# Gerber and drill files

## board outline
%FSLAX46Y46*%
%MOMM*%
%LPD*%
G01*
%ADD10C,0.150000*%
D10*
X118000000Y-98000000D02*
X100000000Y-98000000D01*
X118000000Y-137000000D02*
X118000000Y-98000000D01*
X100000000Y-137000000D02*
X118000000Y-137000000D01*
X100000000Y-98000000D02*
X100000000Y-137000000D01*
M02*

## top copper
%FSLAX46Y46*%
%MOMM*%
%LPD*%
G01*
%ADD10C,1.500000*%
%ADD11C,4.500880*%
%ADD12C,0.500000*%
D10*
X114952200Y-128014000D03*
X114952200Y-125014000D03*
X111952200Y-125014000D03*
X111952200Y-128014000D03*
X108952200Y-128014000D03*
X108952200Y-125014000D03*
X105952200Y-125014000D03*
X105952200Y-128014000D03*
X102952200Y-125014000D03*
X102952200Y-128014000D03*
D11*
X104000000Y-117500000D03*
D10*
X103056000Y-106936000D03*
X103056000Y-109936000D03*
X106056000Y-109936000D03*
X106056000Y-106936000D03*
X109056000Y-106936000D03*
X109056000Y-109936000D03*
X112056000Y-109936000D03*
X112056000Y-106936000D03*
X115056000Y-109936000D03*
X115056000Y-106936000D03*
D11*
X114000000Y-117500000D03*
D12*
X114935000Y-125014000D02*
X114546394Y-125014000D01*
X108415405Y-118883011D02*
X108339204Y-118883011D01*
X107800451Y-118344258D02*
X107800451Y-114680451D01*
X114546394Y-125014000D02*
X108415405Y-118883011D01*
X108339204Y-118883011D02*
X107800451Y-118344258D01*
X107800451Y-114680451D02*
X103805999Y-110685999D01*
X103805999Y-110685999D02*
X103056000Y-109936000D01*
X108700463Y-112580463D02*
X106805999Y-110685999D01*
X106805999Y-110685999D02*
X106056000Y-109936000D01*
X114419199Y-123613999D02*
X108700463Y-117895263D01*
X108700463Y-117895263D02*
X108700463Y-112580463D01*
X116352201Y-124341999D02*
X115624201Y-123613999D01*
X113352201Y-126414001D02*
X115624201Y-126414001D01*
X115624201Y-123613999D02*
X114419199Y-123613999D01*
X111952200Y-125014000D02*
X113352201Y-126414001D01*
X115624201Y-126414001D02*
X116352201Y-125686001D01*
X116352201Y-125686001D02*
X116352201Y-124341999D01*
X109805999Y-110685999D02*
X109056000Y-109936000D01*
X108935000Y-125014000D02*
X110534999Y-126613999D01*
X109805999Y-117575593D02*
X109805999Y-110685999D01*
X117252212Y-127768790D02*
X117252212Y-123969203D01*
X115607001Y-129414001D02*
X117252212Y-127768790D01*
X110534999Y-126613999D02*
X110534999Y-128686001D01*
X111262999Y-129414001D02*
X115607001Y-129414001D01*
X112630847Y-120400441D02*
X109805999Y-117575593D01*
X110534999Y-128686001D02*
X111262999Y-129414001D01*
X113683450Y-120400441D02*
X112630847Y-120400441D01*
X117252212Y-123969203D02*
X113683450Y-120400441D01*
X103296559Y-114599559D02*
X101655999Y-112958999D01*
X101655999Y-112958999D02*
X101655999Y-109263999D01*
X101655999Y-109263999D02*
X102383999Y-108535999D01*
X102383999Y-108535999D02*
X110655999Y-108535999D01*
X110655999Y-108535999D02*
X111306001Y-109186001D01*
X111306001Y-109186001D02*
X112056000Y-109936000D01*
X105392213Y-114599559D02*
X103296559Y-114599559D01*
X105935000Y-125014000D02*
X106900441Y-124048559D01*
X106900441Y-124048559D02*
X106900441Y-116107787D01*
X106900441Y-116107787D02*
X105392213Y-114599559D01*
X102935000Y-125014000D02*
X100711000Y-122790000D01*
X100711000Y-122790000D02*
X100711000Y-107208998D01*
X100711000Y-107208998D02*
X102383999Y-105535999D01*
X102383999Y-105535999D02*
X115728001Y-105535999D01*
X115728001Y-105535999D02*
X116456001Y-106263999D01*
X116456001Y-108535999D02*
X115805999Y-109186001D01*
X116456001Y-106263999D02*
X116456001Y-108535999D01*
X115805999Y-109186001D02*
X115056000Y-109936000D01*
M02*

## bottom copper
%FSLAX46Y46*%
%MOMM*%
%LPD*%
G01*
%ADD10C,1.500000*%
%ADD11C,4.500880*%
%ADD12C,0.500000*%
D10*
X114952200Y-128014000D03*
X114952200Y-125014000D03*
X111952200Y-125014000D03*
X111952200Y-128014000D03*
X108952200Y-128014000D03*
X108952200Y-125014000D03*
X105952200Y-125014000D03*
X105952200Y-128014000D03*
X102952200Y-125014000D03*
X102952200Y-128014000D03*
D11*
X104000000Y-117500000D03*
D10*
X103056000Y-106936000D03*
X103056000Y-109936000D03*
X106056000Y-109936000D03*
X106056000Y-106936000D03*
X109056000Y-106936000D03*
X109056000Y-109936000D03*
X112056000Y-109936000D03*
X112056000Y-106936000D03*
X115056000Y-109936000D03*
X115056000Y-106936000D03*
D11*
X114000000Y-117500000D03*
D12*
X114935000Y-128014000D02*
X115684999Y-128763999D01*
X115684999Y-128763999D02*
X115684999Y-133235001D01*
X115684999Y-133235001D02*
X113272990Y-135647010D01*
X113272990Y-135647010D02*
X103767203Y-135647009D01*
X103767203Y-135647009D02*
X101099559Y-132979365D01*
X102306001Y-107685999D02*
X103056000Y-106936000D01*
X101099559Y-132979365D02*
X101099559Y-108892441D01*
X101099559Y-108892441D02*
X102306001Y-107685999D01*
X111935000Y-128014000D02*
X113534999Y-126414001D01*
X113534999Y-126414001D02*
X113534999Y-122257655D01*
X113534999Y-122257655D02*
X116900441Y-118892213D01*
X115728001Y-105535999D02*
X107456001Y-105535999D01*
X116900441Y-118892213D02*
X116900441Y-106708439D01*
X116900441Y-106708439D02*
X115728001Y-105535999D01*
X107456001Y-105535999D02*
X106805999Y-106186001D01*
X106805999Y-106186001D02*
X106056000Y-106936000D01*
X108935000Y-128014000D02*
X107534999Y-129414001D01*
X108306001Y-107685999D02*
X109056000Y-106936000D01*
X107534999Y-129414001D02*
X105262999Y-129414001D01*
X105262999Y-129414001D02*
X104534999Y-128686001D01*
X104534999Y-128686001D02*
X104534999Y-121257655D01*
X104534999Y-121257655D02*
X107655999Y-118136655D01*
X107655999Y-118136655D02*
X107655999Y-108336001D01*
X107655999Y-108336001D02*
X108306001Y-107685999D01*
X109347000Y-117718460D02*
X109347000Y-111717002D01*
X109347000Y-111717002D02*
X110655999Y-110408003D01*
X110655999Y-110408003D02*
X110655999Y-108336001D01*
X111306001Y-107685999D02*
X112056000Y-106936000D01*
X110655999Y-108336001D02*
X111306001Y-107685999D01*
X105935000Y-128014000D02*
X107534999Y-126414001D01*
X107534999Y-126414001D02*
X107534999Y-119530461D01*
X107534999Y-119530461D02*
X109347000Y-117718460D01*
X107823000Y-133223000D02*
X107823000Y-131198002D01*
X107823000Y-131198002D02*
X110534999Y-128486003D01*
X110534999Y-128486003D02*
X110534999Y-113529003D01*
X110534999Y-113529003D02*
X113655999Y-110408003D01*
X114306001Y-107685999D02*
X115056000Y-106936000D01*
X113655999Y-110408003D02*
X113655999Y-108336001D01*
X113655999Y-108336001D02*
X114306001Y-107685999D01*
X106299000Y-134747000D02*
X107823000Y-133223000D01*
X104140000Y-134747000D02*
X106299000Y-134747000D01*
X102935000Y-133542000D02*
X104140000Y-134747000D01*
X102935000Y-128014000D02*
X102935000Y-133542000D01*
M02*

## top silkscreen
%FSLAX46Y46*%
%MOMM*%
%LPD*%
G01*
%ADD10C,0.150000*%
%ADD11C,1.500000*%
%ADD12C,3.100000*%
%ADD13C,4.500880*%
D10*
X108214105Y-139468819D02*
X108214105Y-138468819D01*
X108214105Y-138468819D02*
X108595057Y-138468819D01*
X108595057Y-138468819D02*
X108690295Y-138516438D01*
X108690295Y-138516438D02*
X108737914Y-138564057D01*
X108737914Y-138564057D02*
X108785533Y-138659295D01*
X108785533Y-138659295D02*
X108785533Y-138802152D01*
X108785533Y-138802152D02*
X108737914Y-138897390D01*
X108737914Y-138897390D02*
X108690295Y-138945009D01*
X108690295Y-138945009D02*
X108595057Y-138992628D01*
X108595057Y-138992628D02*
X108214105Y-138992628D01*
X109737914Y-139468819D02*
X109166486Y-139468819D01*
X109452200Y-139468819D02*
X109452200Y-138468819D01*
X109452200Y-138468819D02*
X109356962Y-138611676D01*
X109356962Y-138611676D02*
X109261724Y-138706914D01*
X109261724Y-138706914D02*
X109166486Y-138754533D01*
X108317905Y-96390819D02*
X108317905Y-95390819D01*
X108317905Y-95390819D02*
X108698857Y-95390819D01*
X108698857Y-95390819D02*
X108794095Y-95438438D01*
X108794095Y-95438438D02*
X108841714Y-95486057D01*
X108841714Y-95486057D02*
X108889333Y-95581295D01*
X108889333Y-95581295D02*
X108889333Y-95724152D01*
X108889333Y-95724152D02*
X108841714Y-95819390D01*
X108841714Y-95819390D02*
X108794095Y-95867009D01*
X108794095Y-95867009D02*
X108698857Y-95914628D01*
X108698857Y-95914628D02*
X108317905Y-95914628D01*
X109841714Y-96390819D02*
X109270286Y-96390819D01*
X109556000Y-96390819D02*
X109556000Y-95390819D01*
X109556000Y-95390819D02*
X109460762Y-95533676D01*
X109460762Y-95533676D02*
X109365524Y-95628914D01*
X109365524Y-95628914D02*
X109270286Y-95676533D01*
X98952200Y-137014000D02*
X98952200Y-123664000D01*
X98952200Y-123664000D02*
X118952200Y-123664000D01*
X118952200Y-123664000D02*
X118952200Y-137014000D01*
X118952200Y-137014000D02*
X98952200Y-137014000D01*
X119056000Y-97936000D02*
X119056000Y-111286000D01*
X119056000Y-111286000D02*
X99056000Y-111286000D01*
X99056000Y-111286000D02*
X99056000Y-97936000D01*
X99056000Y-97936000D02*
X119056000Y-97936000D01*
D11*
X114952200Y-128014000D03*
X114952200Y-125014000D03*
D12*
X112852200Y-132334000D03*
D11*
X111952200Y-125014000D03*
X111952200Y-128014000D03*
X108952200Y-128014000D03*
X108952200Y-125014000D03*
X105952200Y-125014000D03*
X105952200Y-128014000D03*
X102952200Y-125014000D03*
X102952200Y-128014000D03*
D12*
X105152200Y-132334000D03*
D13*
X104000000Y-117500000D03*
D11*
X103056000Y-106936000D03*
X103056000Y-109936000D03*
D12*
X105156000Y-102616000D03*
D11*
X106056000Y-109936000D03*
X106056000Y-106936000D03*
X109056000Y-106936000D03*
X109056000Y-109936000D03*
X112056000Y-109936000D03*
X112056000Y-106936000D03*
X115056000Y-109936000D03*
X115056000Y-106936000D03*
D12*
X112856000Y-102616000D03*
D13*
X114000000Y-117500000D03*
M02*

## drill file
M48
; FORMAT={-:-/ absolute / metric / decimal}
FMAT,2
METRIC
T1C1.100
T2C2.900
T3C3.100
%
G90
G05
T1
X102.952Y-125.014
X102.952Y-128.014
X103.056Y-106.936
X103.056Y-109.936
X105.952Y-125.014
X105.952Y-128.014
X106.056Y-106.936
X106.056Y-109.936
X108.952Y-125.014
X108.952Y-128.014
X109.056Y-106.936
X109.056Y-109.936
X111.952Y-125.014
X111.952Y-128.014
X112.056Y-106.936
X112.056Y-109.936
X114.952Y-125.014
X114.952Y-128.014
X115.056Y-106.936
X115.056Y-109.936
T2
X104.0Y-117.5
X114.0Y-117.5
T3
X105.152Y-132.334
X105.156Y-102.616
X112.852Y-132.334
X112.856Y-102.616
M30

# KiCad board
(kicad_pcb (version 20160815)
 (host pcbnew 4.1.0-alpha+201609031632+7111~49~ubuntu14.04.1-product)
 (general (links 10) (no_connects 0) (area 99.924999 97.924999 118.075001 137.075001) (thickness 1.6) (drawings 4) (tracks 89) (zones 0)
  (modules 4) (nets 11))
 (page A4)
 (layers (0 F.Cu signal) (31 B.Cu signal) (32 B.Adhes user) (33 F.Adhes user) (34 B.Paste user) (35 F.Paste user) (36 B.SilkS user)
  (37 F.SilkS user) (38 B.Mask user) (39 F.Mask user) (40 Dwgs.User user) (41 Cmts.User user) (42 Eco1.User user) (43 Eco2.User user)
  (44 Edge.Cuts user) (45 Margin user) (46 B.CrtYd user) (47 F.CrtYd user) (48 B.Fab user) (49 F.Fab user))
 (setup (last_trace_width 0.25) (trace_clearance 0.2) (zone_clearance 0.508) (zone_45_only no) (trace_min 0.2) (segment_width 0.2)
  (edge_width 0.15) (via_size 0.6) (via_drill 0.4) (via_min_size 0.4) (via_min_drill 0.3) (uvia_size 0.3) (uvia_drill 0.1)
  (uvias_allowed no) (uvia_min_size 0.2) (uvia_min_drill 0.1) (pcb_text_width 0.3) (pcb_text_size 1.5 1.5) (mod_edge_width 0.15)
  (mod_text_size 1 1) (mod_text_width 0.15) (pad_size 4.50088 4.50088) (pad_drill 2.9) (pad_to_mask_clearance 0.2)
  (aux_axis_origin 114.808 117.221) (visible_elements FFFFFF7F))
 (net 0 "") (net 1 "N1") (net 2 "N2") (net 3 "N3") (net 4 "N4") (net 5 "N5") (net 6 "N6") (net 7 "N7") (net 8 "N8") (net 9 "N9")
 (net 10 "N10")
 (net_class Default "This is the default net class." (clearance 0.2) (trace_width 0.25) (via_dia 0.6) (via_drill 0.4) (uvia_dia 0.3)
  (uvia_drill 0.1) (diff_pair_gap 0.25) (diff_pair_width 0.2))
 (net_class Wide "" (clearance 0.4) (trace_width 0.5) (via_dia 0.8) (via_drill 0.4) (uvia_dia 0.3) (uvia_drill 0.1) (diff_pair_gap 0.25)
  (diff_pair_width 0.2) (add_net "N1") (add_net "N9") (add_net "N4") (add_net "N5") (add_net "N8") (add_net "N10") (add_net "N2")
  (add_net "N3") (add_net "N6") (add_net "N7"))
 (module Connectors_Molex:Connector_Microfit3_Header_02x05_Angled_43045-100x (layer F.Cu) (at 114.9522 128.014)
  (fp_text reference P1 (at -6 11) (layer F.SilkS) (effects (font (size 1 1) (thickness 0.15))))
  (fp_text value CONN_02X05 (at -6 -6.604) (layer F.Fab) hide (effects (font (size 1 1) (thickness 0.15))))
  (fp_line (start -16 9) (end -16 -4.35) (layer F.SilkS) (width 0.15))
  (fp_line (start -16 -4.35) (end 4 -4.35) (layer F.SilkS) (width 0.15))
  (fp_line (start 4 -4.35) (end 4 9) (layer F.SilkS) (width 0.15))
  (fp_line (start 4 9) (end -16 9) (layer F.SilkS) (width 0.15))
  (pad 1 thru_hole circle (at 0 0) (size 1.5 1.5) (drill 1.1) (layers *.Cu *.Mask F.SilkS) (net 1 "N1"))
  (pad 6 thru_hole circle (at 0 -3) (size 1.5 1.5) (drill 1.1) (layers *.Cu *.Mask F.SilkS) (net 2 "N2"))
  (pad "" np_thru_hole circle (at -2.1 4.32) (size 3.1 3.1) (drill 3.1) (layers *.Cu *.Mask F.SilkS))
  (pad 7 thru_hole circle (at -3 -3) (size 1.5 1.5) (drill 1.1) (layers *.Cu *.Mask F.SilkS) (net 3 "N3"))
  (pad 2 thru_hole circle (at -3 0) (size 1.5 1.5) (drill 1.1) (layers *.Cu *.Mask F.SilkS) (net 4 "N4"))
  (pad 3 thru_hole circle (at -6 0) (size 1.5 1.5) (drill 1.1) (layers *.Cu *.Mask F.SilkS) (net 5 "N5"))
  (pad 8 thru_hole circle (at -6 -3) (size 1.5 1.5) (drill 1.1) (layers *.Cu *.Mask F.SilkS) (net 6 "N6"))
  (pad 9 thru_hole circle (at -9 -3) (size 1.5 1.5) (drill 1.1) (layers *.Cu *.Mask F.SilkS) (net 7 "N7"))
  (pad 4 thru_hole circle (at -9 0) (size 1.5 1.5) (drill 1.1) (layers *.Cu *.Mask F.SilkS) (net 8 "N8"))
  (pad 10 thru_hole circle (at -12 -3) (size 1.5 1.5) (drill 1.1) (layers *.Cu *.Mask F.SilkS) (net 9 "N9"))
  (pad 5 thru_hole circle (at -12 0) (size 1.5 1.5) (drill 1.1) (layers *.Cu *.Mask F.SilkS) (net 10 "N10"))
  (pad "" np_thru_hole circle (at -9.8 4.32) (size 3.1 3.1) (drill 3.1) (layers *.Cu *.Mask F.SilkS)))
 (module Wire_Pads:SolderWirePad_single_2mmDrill (layer F.Cu) (at 103.632 117.221)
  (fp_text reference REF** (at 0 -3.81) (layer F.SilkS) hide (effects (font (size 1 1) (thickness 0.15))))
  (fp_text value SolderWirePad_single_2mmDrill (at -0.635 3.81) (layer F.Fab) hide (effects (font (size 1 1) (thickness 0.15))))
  (pad 1 thru_hole circle (at 0.368 0.279) (size 4.50088 4.50088) (drill 2.9) (layers *.Cu *.Mask F.SilkS)))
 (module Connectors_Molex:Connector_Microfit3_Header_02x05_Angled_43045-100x (layer F.Cu) (at 103.056 106.936 180)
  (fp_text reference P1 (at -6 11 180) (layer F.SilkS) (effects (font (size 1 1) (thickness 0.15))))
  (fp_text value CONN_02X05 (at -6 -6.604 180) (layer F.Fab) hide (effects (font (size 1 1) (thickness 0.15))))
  (fp_line (start -16 9) (end -16 -4.35) (layer F.SilkS) (width 0.15))
  (fp_line (start -16 -4.35) (end 4 -4.35) (layer F.SilkS) (width 0.15))
  (fp_line (start 4 -4.35) (end 4 9) (layer F.SilkS) (width 0.15))
  (fp_line (start 4 9) (end -16 9) (layer F.SilkS) (width 0.15))
  (pad 1 thru_hole circle (at 0 0 180) (size 1.5 1.5) (drill 1.1) (layers *.Cu *.Mask F.SilkS) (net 1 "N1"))
  (pad 6 thru_hole circle (at 0 -3 180) (size 1.5 1.5) (drill 1.1) (layers *.Cu *.Mask F.SilkS) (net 2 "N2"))
  (pad "" np_thru_hole circle (at -2.1 4.32 180) (size 3.1 3.1) (drill 3.1) (layers *.Cu *.Mask F.SilkS))
  (pad 7 thru_hole circle (at -3 -3 180) (size 1.5 1.5) (drill 1.1) (layers *.Cu *.Mask F.SilkS) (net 3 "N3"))
  (pad 2 thru_hole circle (at -3 0 180) (size 1.5 1.5) (drill 1.1) (layers *.Cu *.Mask F.SilkS) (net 4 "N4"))
  (pad 3 thru_hole circle (at -6 0 180) (size 1.5 1.5) (drill 1.1) (layers *.Cu *.Mask F.SilkS) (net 5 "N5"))
  (pad 8 thru_hole circle (at -6 -3 180) (size 1.5 1.5) (drill 1.1) (layers *.Cu *.Mask F.SilkS) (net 6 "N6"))
  (pad 9 thru_hole circle (at -9 -3 180) (size 1.5 1.5) (drill 1.1) (layers *.Cu *.Mask F.SilkS) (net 7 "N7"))
  (pad 4 thru_hole circle (at -9 0 180) (size 1.5 1.5) (drill 1.1) (layers *.Cu *.Mask F.SilkS) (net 8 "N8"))
  (pad 10 thru_hole circle (at -12 -3 180) (size 1.5 1.5) (drill 1.1) (layers *.Cu *.Mask F.SilkS) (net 9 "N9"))
  (pad 5 thru_hole circle (at -12 0 180) (size 1.5 1.5) (drill 1.1) (layers *.Cu *.Mask F.SilkS) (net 10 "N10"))
  (pad "" np_thru_hole circle (at -9.8 4.32 180) (size 3.1 3.1) (drill 3.1) (layers *.Cu *.Mask F.SilkS)))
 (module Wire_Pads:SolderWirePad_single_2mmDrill (layer F.Cu) (at 114.808 117.348)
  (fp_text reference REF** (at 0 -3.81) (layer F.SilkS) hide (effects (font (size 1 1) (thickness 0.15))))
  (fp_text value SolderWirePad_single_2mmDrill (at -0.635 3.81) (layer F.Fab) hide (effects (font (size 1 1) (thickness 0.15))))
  (pad 1 thru_hole circle (at -0.808 0.152) (size 4.50088 4.50088) (drill 2.9) (layers *.Cu *.Mask F.SilkS)))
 (gr_line (start 118 98) (end 100 98) (angle 90) (layer Edge.Cuts) (width 0.15))
 (gr_line (start 118 137) (end 118 98) (angle 90) (layer Edge.Cuts) (width 0.15))
 (gr_line (start 100 137) (end 118 137) (angle 90) (layer Edge.Cuts) (width 0.15))
 (gr_line (start 100 98) (end 100 137) (angle 90) (layer Edge.Cuts) (width 0.15))
 (segment (start 114.935 128.014) (end 115.684999 128.763999) (width 0.5) (layer B.Cu) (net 1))
 (segment (start 115.684999 128.763999) (end 115.684999 133.235001) (width 0.5) (layer B.Cu) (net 1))
 (segment (start 115.684999 133.235001) (end 113.27299 135.64701) (width 0.5) (layer B.Cu) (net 1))
 (segment (start 113.27299 135.64701) (end 103.767203 135.647009) (width 0.5) (layer B.Cu) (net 1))
 (segment (start 103.767203 135.647009) (end 101.099559 132.979365) (width 0.5) (layer B.Cu) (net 1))
 (segment (start 102.306001 107.685999) (end 103.056 106.936) (width 0.5) (layer B.Cu) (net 1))
 (segment (start 101.099559 132.979365) (end 101.099559 108.892441) (width 0.5) (layer B.Cu) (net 1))
 (segment (start 101.099559 108.892441) (end 102.306001 107.685999) (width 0.5) (layer B.Cu) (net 1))
 (segment (start 114.935 125.014) (end 114.546394 125.014) (width 0.5) (layer F.Cu) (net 2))
 (segment (start 108.415405 118.883011) (end 108.339204 118.883011) (width 0.5) (layer F.Cu) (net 2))
 (segment (start 107.800451 118.344258) (end 107.800451 114.680451) (width 0.5) (layer F.Cu) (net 2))
 (segment (start 114.546394 125.014) (end 108.415405 118.883011) (width 0.5) (layer F.Cu) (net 2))
 (segment (start 108.339204 118.883011) (end 107.800451 118.344258) (width 0.5) (layer F.Cu) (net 2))
 (segment (start 107.800451 114.680451) (end 103.805999 110.685999) (width 0.5) (layer F.Cu) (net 2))
 (segment (start 103.805999 110.685999) (end 103.056 109.936) (width 0.5) (layer F.Cu) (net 2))
 (segment (start 108.700463 112.580463) (end 106.805999 110.685999) (width 0.5) (layer F.Cu) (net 3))
 (segment (start 106.805999 110.685999) (end 106.056 109.936) (width 0.5) (layer F.Cu) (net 3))
 (segment (start 114.419199 123.613999) (end 108.700463 117.895263) (width 0.5) (layer F.Cu) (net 3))
 (segment (start 108.700463 117.895263) (end 108.700463 112.580463) (width 0.5) (layer F.Cu) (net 3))
 (segment (start 116.352201 124.341999) (end 115.624201 123.613999) (width 0.5) (layer F.Cu) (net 3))
 (segment (start 113.352201 126.414001) (end 115.624201 126.414001) (width 0.5) (layer F.Cu) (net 3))
 (segment (start 115.624201 123.613999) (end 114.419199 123.613999) (width 0.5) (layer F.Cu) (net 3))
 (segment (start 111.9522 125.014) (end 113.352201 126.414001) (width 0.5) (layer F.Cu) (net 3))
 (segment (start 115.624201 126.414001) (end 116.352201 125.686001) (width 0.5) (layer F.Cu) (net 3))
 (segment (start 116.352201 125.686001) (end 116.352201 124.341999) (width 0.5) (layer F.Cu) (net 3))
 (segment (start 111.935 128.014) (end 113.534999 126.414001) (width 0.5) (layer B.Cu) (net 4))
 (segment (start 113.534999 126.414001) (end 113.534999 122.257655) (width 0.5) (layer B.Cu) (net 4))
 (segment (start 113.534999 122.257655) (end 116.900441 118.892213) (width 0.5) (layer B.Cu) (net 4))
 (segment (start 115.728001 105.535999) (end 107.456001 105.535999) (width 0.5) (layer B.Cu) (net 4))
 (segment (start 116.900441 118.892213) (end 116.900441 106.708439) (width 0.5) (layer B.Cu) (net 4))
 (segment (start 116.900441 106.708439) (end 115.728001 105.535999) (width 0.5) (layer B.Cu) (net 4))
 (segment (start 107.456001 105.535999) (end 106.805999 106.186001) (width 0.5) (layer B.Cu) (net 4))
 (segment (start 106.805999 106.186001) (end 106.056 106.936) (width 0.5) (layer B.Cu) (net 4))
 (segment (start 108.935 128.014) (end 107.534999 129.414001) (width 0.5) (layer B.Cu) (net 5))
 (segment (start 108.306001 107.685999) (end 109.056 106.936) (width 0.5) (layer B.Cu) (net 5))
 (segment (start 107.534999 129.414001) (end 105.262999 129.414001) (width 0.5) (layer B.Cu) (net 5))
 (segment (start 105.262999 129.414001) (end 104.534999 128.686001) (width 0.5) (layer B.Cu) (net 5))
 (segment (start 104.534999 128.686001) (end 104.534999 121.257655) (width 0.5) (layer B.Cu) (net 5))
 (segment (start 104.534999 121.257655) (end 107.655999 118.136655) (width 0.5) (layer B.Cu) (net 5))
 (segment (start 107.655999 118.136655) (end 107.655999 108.336001) (width 0.5) (layer B.Cu) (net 5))
 (segment (start 107.655999 108.336001) (end 108.306001 107.685999) (width 0.5) (layer B.Cu) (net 5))
 (segment (start 109.805999 110.685999) (end 109.056 109.936) (width 0.5) (layer F.Cu) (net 6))
 (segment (start 108.935 125.014) (end 110.534999 126.613999) (width 0.5) (layer F.Cu) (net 6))
 (segment (start 109.805999 117.575593) (end 109.805999 110.685999) (width 0.5) (layer F.Cu) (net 6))
 (segment (start 117.252212 127.76879) (end 117.252212 123.969203) (width 0.5) (layer F.Cu) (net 6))
 (segment (start 115.607001 129.414001) (end 117.252212 127.76879) (width 0.5) (layer F.Cu) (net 6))
 (segment (start 110.534999 126.613999) (end 110.534999 128.686001) (width 0.5) (layer F.Cu) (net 6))
 (segment (start 111.262999 129.414001) (end 115.607001 129.414001) (width 0.5) (layer F.Cu) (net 6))
 (segment (start 112.630847 120.400441) (end 109.805999 117.575593) (width 0.5) (layer F.Cu) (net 6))
 (segment (start 110.534999 128.686001) (end 111.262999 129.414001) (width 0.5) (layer F.Cu) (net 6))
 (segment (start 113.68345 120.400441) (end 112.630847 120.400441) (width 0.5) (layer F.Cu) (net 6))
 (segment (start 117.252212 123.969203) (end 113.68345 120.400441) (width 0.5) (layer F.Cu) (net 6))
 (segment (start 103.296559 114.599559) (end 101.655999 112.958999) (width 0.5) (layer F.Cu) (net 7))
 (segment (start 101.655999 112.958999) (end 101.655999 109.263999) (width 0.5) (layer F.Cu) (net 7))
 (segment (start 101.655999 109.263999) (end 102.383999 108.535999) (width 0.5) (layer F.Cu) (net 7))
 (segment (start 102.383999 108.535999) (end 110.655999 108.535999) (width 0.5) (layer F.Cu) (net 7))
 (segment (start 110.655999 108.535999) (end 111.306001 109.186001) (width 0.5) (layer F.Cu) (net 7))
 (segment (start 111.306001 109.186001) (end 112.056 109.936) (width 0.5) (layer F.Cu) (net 7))
 (segment (start 105.392213 114.599559) (end 103.296559 114.599559) (width 0.5) (layer F.Cu) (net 7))
 (segment (start 105.935 125.014) (end 106.900441 124.048559) (width 0.5) (layer F.Cu) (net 7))
 (segment (start 106.900441 124.048559) (end 106.900441 116.107787) (width 0.5) (layer F.Cu) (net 7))
 (segment (start 106.900441 116.107787) (end 105.392213 114.599559) (width 0.5) (layer F.Cu) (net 7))
 (segment (start 109.347 117.71846) (end 109.347 111.717002) (width 0.5) (layer B.Cu) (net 8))
 (segment (start 109.347 111.717002) (end 110.655999 110.408003) (width 0.5) (layer B.Cu) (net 8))
 (segment (start 110.655999 110.408003) (end 110.655999 108.336001) (width 0.5) (layer B.Cu) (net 8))
 (segment (start 111.306001 107.685999) (end 112.056 106.936) (width 0.5) (layer B.Cu) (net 8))
 (segment (start 110.655999 108.336001) (end 111.306001 107.685999) (width 0.5) (layer B.Cu) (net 8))
 (segment (start 105.935 128.014) (end 107.534999 126.414001) (width 0.5) (layer B.Cu) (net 8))
 (segment (start 107.534999 126.414001) (end 107.534999 119.530461) (width 0.5) (layer B.Cu) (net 8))
 (segment (start 107.534999 119.530461) (end 109.347 117.71846) (width 0.5) (layer B.Cu) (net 8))
 (segment (start 102.935 125.014) (end 100.711 122.79) (width 0.5) (layer F.Cu) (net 9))
 (segment (start 100.711 122.79) (end 100.711 107.208998) (width 0.5) (layer F.Cu) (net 9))
 (segment (start 100.711 107.208998) (end 102.383999 105.535999) (width 0.5) (layer F.Cu) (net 9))
 (segment (start 102.383999 105.535999) (end 115.728001 105.535999) (width 0.5) (layer F.Cu) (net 9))
 (segment (start 115.728001 105.535999) (end 116.456001 106.263999) (width 0.5) (layer F.Cu) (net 9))
 (segment (start 116.456001 108.535999) (end 115.805999 109.186001) (width 0.5) (layer F.Cu) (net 9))
 (segment (start 116.456001 106.263999) (end 116.456001 108.535999) (width 0.5) (layer F.Cu) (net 9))
 (segment (start 115.805999 109.186001) (end 115.056 109.936) (width 0.5) (layer F.Cu) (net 9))
 (segment (start 107.823 133.223) (end 107.823 131.198002) (width 0.5) (layer B.Cu) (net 10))
 (segment (start 107.823 131.198002) (end 110.534999 128.486003) (width 0.5) (layer B.Cu) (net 10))
 (segment (start 110.534999 128.486003) (end 110.534999 113.529003) (width 0.5) (layer B.Cu) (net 10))
 (segment (start 110.534999 113.529003) (end 113.655999 110.408003) (width 0.5) (layer B.Cu) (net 10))
 (segment (start 114.306001 107.685999) (end 115.056 106.936) (width 0.5) (layer B.Cu) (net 10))
 (segment (start 113.655999 110.408003) (end 113.655999 108.336001) (width 0.5) (layer B.Cu) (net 10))
 (segment (start 113.655999 108.336001) (end 114.306001 107.685999) (width 0.5) (layer B.Cu) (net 10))
 (segment (start 106.299 134.747) (end 107.823 133.223) (width 0.5) (layer B.Cu) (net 10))
 (segment (start 104.14 134.747) (end 106.299 134.747) (width 0.5) (layer B.Cu) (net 10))
 (segment (start 102.935 133.542) (end 104.14 134.747) (width 0.5) (layer B.Cu) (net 10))
 (segment (start 102.935 128.014) (end 102.935 133.542) (width 0.5) (layer B.Cu) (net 10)))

